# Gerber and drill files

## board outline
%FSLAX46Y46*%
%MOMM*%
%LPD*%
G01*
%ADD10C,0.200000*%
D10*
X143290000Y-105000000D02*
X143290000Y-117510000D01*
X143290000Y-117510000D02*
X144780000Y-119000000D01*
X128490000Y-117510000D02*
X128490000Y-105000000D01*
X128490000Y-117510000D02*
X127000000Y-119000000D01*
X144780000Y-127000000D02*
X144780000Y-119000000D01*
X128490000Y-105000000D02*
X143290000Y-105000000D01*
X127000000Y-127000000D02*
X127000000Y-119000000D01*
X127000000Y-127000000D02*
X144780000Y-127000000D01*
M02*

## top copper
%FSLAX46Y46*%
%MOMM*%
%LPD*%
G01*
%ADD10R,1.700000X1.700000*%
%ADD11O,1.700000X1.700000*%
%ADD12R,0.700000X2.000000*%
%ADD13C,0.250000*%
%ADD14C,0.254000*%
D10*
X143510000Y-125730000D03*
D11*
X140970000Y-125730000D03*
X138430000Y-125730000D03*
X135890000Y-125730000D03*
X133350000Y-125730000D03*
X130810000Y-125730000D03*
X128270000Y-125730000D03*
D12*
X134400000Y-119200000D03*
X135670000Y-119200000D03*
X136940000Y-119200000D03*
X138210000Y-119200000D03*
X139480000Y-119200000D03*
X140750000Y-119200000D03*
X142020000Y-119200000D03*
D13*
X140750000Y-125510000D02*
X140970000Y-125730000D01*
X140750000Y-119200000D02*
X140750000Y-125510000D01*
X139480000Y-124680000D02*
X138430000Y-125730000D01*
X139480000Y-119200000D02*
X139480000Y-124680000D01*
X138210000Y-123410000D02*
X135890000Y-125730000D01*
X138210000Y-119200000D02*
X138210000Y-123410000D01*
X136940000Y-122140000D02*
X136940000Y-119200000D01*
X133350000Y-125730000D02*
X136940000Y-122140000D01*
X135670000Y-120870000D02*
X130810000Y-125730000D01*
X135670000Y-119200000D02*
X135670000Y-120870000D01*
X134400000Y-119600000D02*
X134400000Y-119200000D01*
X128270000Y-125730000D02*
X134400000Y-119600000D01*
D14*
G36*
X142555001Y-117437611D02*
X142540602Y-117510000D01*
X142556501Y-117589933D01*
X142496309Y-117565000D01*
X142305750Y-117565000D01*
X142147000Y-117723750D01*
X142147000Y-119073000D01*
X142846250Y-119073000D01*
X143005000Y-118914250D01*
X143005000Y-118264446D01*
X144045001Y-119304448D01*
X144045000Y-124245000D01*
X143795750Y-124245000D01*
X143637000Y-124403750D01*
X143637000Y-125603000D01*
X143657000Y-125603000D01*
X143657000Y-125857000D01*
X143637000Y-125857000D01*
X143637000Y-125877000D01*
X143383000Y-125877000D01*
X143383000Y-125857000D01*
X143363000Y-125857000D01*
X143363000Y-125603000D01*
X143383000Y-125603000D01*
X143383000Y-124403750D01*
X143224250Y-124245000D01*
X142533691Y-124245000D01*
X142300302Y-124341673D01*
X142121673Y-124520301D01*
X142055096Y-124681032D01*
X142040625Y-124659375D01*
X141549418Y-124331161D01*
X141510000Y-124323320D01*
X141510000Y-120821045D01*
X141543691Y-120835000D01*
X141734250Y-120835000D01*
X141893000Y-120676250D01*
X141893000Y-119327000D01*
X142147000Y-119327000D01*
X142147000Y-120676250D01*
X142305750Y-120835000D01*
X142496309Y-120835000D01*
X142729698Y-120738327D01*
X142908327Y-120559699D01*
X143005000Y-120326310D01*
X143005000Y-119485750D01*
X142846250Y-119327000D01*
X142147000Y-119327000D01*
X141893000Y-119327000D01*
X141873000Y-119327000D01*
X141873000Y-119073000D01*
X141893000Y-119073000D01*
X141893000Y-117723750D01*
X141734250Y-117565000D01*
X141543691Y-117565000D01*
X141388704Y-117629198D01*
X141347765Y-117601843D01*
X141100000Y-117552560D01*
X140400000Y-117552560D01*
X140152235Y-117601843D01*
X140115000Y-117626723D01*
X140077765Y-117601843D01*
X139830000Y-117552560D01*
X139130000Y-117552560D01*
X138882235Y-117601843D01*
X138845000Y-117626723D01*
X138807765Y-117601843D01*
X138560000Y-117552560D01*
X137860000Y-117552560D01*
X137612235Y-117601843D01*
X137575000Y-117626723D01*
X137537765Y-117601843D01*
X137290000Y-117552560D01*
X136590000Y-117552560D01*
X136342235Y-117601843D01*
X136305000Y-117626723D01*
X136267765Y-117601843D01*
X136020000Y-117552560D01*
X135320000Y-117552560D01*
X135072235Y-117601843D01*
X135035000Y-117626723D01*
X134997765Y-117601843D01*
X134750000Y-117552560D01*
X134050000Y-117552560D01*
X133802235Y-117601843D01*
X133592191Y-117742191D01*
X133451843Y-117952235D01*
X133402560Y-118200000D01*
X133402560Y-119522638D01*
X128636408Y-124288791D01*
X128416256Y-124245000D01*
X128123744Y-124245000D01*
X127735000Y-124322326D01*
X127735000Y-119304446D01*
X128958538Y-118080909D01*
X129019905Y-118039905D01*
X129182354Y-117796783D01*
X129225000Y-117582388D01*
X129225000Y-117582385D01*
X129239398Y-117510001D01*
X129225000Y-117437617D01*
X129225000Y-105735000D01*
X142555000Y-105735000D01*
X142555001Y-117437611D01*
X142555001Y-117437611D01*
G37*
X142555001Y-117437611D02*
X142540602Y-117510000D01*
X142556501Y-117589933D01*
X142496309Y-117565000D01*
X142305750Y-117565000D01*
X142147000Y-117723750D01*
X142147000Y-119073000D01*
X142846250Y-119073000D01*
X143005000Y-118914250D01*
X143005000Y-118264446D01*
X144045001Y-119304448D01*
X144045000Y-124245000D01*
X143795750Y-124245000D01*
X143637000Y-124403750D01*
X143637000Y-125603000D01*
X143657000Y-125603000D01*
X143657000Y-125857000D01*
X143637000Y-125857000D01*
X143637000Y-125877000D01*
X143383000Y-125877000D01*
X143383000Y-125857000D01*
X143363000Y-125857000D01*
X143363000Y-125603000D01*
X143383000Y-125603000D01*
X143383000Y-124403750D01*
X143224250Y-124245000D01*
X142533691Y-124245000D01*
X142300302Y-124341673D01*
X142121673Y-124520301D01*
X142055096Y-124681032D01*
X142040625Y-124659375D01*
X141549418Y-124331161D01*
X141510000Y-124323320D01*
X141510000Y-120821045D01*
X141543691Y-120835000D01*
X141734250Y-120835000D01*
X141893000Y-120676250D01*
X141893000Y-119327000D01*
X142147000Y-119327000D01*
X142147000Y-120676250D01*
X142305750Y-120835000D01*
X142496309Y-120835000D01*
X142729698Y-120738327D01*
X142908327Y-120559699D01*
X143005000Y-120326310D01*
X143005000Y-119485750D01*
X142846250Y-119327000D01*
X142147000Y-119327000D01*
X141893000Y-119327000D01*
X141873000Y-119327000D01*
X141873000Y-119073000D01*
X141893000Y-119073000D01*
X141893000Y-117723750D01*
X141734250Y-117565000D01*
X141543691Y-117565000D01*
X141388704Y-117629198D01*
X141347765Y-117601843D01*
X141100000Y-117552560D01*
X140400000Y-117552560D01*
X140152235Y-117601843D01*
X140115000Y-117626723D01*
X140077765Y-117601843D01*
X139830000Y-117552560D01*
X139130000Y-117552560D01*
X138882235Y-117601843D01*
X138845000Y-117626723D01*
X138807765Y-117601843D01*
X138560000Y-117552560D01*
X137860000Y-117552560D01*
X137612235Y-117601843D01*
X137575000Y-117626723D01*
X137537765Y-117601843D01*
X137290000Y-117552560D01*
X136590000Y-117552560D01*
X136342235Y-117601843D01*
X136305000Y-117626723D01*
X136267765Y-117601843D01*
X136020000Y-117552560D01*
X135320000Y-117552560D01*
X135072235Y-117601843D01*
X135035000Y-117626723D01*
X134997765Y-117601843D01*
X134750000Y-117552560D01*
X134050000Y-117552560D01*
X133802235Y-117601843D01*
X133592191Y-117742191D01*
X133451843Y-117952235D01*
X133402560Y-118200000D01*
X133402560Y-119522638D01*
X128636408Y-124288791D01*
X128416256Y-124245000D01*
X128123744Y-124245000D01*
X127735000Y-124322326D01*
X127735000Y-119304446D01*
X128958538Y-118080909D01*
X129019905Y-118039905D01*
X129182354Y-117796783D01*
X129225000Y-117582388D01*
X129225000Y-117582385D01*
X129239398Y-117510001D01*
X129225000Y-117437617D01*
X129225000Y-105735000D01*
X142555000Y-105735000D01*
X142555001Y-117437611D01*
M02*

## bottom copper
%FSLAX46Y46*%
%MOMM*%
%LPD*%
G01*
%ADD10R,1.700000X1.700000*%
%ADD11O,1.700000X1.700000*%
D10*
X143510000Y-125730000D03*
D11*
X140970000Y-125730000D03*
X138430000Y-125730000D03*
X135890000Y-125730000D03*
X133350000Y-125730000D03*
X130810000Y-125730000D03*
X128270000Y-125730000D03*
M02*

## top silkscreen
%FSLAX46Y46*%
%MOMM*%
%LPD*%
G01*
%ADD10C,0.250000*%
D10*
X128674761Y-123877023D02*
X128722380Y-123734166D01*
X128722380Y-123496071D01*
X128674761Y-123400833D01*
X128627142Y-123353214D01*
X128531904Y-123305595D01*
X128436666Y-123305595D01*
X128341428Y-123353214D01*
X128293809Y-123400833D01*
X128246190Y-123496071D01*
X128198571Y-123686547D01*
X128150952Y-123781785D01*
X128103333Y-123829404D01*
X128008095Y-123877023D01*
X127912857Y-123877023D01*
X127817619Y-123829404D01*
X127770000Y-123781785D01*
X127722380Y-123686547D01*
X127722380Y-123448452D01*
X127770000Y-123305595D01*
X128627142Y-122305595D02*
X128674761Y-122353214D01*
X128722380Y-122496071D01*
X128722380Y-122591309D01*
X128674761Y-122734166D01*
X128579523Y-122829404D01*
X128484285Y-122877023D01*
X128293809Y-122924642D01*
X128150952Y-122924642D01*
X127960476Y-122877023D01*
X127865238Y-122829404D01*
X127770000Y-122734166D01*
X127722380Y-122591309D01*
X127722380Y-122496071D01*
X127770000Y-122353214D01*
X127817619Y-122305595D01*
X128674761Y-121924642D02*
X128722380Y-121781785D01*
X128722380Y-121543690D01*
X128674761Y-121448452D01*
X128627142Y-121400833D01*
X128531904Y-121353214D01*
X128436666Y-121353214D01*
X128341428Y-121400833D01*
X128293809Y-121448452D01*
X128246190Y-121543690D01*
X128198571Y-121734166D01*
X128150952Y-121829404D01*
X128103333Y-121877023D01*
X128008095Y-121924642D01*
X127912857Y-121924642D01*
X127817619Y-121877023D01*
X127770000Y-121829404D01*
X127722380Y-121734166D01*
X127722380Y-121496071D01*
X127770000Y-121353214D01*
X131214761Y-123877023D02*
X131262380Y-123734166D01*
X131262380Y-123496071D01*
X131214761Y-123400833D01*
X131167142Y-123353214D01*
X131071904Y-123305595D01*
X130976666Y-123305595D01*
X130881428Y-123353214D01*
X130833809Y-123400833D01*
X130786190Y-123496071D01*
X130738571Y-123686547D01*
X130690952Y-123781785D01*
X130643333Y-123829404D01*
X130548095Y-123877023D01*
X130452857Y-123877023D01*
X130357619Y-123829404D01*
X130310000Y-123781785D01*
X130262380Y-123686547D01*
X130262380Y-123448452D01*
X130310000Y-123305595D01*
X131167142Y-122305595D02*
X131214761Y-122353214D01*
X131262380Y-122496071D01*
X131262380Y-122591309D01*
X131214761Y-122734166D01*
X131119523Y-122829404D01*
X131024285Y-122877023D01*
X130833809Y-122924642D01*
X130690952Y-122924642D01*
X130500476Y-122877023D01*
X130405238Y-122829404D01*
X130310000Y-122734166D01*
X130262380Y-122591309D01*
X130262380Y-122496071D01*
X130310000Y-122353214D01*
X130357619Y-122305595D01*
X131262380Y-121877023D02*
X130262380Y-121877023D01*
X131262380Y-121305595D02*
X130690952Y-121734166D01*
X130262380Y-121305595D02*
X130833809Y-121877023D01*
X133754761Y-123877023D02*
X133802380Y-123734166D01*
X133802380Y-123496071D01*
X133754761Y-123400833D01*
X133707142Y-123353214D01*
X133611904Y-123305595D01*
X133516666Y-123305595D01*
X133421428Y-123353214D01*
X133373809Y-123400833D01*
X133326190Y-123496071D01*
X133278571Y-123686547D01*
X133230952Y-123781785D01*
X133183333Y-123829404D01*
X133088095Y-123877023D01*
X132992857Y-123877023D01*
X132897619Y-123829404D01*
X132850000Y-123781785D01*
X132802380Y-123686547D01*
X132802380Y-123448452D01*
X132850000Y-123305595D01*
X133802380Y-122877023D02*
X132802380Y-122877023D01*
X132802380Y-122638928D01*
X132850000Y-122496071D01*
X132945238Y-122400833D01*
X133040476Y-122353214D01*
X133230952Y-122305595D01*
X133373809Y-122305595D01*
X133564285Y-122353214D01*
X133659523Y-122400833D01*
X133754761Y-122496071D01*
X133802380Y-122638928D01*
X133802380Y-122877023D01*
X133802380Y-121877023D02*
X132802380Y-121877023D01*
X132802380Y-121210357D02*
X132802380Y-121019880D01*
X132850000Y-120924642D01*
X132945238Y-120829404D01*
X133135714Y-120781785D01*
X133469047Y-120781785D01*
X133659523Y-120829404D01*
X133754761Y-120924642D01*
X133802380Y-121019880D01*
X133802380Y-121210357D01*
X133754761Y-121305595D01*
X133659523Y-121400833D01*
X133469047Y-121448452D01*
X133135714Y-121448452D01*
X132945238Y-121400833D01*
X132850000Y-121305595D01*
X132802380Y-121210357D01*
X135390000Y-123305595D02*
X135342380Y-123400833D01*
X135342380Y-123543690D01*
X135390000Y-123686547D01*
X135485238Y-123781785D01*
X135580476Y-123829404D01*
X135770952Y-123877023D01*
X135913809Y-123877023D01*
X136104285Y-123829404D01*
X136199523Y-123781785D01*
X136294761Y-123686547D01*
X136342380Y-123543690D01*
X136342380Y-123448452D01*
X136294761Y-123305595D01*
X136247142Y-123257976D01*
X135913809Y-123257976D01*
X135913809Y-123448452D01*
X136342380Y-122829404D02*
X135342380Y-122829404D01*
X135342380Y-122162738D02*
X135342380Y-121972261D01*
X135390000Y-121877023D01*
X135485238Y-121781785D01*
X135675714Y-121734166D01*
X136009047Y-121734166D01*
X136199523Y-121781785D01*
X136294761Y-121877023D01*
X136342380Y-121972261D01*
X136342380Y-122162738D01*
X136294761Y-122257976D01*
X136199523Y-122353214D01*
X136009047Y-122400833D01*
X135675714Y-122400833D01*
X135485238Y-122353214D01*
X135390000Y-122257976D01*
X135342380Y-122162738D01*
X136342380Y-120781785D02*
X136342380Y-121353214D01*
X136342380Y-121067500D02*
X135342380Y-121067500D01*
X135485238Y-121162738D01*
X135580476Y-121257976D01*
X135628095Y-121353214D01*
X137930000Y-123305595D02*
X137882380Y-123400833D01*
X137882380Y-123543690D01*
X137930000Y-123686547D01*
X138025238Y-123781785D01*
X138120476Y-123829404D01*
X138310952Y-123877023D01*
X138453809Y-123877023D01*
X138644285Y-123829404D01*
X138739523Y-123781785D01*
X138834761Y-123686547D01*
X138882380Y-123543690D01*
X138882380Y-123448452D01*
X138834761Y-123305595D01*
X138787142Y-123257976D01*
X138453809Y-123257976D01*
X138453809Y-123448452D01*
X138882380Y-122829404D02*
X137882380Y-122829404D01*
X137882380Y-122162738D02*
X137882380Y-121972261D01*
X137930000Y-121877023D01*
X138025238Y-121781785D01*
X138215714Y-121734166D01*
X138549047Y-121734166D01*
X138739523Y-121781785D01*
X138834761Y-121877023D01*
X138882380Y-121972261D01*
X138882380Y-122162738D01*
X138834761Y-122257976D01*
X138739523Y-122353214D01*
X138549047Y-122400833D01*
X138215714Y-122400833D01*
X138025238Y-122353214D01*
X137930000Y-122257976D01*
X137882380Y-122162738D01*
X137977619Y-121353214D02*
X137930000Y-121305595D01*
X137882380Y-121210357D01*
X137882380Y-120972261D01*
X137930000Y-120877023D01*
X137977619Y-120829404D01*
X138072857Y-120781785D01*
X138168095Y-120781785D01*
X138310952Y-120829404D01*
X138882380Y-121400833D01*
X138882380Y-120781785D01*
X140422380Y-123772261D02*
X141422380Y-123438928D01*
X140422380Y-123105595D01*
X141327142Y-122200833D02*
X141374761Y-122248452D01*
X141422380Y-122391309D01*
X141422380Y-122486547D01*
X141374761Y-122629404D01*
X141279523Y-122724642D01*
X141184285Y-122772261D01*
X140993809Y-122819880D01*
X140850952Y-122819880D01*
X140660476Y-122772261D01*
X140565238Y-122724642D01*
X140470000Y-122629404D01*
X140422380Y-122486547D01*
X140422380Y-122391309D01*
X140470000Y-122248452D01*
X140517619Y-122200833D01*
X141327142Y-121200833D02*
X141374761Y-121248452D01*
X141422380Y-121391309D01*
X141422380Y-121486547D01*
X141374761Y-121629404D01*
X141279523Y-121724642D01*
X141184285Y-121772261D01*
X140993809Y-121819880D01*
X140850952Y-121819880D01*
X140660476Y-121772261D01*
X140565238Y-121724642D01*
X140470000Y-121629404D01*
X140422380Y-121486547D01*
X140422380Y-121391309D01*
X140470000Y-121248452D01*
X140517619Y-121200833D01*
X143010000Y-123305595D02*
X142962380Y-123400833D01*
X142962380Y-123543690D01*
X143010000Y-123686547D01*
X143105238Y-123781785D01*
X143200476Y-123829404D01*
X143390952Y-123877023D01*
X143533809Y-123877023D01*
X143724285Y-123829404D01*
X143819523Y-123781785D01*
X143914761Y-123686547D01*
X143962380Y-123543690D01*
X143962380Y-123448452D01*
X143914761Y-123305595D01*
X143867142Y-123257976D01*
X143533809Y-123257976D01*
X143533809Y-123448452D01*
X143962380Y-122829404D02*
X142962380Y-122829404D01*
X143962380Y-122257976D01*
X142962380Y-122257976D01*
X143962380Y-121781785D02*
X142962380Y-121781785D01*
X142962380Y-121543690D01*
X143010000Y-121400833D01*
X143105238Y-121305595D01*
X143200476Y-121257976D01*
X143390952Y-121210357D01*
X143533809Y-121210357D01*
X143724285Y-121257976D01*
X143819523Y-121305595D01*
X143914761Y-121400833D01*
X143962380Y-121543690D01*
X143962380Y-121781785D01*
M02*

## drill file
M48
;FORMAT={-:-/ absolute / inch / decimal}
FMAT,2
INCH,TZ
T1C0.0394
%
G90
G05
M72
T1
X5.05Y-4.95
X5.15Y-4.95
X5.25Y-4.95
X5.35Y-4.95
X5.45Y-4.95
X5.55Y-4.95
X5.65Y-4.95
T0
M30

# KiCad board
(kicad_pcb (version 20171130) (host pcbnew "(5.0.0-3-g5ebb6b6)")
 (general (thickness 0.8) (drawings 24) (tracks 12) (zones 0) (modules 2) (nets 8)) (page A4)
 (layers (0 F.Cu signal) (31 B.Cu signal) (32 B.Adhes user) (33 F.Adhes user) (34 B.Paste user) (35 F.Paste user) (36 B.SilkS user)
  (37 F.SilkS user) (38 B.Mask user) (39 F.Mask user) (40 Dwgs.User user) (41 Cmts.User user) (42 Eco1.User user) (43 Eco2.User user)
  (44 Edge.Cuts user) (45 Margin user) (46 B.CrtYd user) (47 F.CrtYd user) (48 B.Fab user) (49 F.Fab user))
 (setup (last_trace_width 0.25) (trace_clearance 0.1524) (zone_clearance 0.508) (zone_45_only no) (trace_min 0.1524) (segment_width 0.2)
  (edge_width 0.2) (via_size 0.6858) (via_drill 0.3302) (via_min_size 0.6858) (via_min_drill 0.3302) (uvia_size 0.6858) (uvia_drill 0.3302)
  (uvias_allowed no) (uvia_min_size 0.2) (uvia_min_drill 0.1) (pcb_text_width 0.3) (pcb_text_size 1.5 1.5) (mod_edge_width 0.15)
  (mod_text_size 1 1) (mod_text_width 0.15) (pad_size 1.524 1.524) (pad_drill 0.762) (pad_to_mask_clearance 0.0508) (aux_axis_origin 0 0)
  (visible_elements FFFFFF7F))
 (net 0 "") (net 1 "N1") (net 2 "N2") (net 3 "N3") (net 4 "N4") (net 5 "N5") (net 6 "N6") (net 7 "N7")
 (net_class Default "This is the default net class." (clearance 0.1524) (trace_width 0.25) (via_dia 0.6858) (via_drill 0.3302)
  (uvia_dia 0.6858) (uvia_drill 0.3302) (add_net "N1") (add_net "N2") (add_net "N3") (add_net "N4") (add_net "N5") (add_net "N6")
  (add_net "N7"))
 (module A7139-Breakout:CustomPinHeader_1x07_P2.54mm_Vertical (layer F.Cu) (at 143.51 125.73 270)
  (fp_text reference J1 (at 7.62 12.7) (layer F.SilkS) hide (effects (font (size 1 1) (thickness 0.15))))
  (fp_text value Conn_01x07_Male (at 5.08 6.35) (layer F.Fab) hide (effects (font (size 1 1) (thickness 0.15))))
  (pad 1 thru_hole rect (at 0 0) (size 1.7 1.7) (drill 1) (layers *.Cu *.Mask) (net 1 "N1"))
  (pad 2 thru_hole oval (at 0 2.54) (size 1.7 1.7) (drill 1) (layers *.Cu *.Mask) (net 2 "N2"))
  (pad 3 thru_hole oval (at 0 5.08 270) (size 1.7 1.7) (drill 1) (layers *.Cu *.Mask) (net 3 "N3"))
  (pad 4 thru_hole oval (at 0 7.62 270) (size 1.7 1.7) (drill 1) (layers *.Cu *.Mask) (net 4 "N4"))
  (pad 5 thru_hole oval (at 0 10.16 270) (size 1.7 1.7) (drill 1) (layers *.Cu *.Mask) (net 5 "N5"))
  (pad 6 thru_hole oval (at 0 12.7 270) (size 1.7 1.7) (drill 1) (layers *.Cu *.Mask) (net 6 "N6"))
  (pad 7 thru_hole oval (at 0 15.24 270) (size 1.7 1.7) (drill 1) (layers *.Cu *.Mask) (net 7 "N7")))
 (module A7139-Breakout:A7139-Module (layer F.Cu) (at 128.49 118.2)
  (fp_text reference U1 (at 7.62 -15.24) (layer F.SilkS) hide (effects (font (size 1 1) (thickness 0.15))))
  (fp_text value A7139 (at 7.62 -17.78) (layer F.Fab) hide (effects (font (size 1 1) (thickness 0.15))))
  (pad 7 smd rect (at 5.91 1) (size 0.7 2) (layers F.Cu F.Paste F.Mask) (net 7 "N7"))
  (pad 6 smd rect (at 7.18 1) (size 0.7 2) (layers F.Cu F.Paste F.Mask) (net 6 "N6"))
  (pad 5 smd rect (at 8.45 1) (size 0.7 2) (layers F.Cu F.Paste F.Mask) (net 5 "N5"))
  (pad 4 smd rect (at 9.72 1) (size 0.7 2) (layers F.Cu F.Paste F.Mask) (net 4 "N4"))
  (pad 3 smd rect (at 10.99 1) (size 0.7 2) (layers F.Cu F.Paste F.Mask) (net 3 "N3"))
  (pad 2 smd rect (at 12.26 1) (size 0.7 2) (layers F.Cu F.Paste F.Mask) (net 2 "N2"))
  (pad 1 smd rect (at 13.53 1) (size 0.7 2) (layers F.Cu F.Paste F.Mask) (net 1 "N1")))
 (gr_line (start 143.29 105) (end 143.29 117.51) (layer Edge.Cuts) (width 0.2))
 (gr_line (start 143.29 117.51) (end 144.78 119) (layer Edge.Cuts) (width 0.2))
 (gr_line (start 128.49 117.51) (end 128.49 105) (layer Edge.Cuts) (width 0.2))
 (gr_line (start 128.49 117.51) (end 127 119) (layer Edge.Cuts) (width 0.2))
 (gr_line (start 144.78 127) (end 144.78 119) (layer Edge.Cuts) (width 0.2))
 (gr_line (start 128.49 105) (end 143.29 105) (layer Edge.Cuts) (width 0.2))
 (gr_line (start 127 127) (end 127 119) (layer Edge.Cuts) (width 0.2))
 (gr_line (start 127 127) (end 144.78 127) (layer Edge.Cuts) (width 0.2))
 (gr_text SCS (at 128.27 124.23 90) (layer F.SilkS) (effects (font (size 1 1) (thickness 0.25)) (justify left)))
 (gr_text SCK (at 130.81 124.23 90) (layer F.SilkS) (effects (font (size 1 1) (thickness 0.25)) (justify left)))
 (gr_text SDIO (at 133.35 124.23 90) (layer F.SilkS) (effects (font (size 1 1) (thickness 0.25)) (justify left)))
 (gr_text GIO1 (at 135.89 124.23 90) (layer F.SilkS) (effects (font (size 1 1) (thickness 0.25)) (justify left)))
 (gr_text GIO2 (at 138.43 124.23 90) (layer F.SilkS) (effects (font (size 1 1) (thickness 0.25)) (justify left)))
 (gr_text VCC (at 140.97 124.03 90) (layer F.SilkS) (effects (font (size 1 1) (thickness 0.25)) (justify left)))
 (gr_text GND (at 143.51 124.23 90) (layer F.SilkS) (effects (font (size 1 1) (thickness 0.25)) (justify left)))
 (segment (start 140.75 125.51) (end 140.97 125.73) (width 0.25) (layer F.Cu) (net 2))
 (segment (start 140.75 119.2) (end 140.75 125.51) (width 0.25) (layer F.Cu) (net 2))
 (segment (start 139.48 124.68) (end 138.43 125.73) (width 0.25) (layer F.Cu) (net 3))
 (segment (start 139.48 119.2) (end 139.48 124.68) (width 0.25) (layer F.Cu) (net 3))
 (segment (start 138.21 123.41) (end 135.89 125.73) (width 0.25) (layer F.Cu) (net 4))
 (segment (start 138.21 119.2) (end 138.21 123.41) (width 0.25) (layer F.Cu) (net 4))
 (segment (start 136.94 122.14) (end 136.94 119.2) (width 0.25) (layer F.Cu) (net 5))
 (segment (start 133.35 125.73) (end 136.94 122.14) (width 0.25) (layer F.Cu) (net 5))
 (segment (start 135.67 120.87) (end 130.81 125.73) (width 0.25) (layer F.Cu) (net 6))
 (segment (start 135.67 119.2) (end 135.67 120.87) (width 0.25) (layer F.Cu) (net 6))
 (segment (start 134.4 119.6) (end 134.4 119.2) (width 0.25) (layer F.Cu) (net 7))
 (segment (start 128.27 125.73) (end 134.4 119.6) (width 0.25) (layer F.Cu) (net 7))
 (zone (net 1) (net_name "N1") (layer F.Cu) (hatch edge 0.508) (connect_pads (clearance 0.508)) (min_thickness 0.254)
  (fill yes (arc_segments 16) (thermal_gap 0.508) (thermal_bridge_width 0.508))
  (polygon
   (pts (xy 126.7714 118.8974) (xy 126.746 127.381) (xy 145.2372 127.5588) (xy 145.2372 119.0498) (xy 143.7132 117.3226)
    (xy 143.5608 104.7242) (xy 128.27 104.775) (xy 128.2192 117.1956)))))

